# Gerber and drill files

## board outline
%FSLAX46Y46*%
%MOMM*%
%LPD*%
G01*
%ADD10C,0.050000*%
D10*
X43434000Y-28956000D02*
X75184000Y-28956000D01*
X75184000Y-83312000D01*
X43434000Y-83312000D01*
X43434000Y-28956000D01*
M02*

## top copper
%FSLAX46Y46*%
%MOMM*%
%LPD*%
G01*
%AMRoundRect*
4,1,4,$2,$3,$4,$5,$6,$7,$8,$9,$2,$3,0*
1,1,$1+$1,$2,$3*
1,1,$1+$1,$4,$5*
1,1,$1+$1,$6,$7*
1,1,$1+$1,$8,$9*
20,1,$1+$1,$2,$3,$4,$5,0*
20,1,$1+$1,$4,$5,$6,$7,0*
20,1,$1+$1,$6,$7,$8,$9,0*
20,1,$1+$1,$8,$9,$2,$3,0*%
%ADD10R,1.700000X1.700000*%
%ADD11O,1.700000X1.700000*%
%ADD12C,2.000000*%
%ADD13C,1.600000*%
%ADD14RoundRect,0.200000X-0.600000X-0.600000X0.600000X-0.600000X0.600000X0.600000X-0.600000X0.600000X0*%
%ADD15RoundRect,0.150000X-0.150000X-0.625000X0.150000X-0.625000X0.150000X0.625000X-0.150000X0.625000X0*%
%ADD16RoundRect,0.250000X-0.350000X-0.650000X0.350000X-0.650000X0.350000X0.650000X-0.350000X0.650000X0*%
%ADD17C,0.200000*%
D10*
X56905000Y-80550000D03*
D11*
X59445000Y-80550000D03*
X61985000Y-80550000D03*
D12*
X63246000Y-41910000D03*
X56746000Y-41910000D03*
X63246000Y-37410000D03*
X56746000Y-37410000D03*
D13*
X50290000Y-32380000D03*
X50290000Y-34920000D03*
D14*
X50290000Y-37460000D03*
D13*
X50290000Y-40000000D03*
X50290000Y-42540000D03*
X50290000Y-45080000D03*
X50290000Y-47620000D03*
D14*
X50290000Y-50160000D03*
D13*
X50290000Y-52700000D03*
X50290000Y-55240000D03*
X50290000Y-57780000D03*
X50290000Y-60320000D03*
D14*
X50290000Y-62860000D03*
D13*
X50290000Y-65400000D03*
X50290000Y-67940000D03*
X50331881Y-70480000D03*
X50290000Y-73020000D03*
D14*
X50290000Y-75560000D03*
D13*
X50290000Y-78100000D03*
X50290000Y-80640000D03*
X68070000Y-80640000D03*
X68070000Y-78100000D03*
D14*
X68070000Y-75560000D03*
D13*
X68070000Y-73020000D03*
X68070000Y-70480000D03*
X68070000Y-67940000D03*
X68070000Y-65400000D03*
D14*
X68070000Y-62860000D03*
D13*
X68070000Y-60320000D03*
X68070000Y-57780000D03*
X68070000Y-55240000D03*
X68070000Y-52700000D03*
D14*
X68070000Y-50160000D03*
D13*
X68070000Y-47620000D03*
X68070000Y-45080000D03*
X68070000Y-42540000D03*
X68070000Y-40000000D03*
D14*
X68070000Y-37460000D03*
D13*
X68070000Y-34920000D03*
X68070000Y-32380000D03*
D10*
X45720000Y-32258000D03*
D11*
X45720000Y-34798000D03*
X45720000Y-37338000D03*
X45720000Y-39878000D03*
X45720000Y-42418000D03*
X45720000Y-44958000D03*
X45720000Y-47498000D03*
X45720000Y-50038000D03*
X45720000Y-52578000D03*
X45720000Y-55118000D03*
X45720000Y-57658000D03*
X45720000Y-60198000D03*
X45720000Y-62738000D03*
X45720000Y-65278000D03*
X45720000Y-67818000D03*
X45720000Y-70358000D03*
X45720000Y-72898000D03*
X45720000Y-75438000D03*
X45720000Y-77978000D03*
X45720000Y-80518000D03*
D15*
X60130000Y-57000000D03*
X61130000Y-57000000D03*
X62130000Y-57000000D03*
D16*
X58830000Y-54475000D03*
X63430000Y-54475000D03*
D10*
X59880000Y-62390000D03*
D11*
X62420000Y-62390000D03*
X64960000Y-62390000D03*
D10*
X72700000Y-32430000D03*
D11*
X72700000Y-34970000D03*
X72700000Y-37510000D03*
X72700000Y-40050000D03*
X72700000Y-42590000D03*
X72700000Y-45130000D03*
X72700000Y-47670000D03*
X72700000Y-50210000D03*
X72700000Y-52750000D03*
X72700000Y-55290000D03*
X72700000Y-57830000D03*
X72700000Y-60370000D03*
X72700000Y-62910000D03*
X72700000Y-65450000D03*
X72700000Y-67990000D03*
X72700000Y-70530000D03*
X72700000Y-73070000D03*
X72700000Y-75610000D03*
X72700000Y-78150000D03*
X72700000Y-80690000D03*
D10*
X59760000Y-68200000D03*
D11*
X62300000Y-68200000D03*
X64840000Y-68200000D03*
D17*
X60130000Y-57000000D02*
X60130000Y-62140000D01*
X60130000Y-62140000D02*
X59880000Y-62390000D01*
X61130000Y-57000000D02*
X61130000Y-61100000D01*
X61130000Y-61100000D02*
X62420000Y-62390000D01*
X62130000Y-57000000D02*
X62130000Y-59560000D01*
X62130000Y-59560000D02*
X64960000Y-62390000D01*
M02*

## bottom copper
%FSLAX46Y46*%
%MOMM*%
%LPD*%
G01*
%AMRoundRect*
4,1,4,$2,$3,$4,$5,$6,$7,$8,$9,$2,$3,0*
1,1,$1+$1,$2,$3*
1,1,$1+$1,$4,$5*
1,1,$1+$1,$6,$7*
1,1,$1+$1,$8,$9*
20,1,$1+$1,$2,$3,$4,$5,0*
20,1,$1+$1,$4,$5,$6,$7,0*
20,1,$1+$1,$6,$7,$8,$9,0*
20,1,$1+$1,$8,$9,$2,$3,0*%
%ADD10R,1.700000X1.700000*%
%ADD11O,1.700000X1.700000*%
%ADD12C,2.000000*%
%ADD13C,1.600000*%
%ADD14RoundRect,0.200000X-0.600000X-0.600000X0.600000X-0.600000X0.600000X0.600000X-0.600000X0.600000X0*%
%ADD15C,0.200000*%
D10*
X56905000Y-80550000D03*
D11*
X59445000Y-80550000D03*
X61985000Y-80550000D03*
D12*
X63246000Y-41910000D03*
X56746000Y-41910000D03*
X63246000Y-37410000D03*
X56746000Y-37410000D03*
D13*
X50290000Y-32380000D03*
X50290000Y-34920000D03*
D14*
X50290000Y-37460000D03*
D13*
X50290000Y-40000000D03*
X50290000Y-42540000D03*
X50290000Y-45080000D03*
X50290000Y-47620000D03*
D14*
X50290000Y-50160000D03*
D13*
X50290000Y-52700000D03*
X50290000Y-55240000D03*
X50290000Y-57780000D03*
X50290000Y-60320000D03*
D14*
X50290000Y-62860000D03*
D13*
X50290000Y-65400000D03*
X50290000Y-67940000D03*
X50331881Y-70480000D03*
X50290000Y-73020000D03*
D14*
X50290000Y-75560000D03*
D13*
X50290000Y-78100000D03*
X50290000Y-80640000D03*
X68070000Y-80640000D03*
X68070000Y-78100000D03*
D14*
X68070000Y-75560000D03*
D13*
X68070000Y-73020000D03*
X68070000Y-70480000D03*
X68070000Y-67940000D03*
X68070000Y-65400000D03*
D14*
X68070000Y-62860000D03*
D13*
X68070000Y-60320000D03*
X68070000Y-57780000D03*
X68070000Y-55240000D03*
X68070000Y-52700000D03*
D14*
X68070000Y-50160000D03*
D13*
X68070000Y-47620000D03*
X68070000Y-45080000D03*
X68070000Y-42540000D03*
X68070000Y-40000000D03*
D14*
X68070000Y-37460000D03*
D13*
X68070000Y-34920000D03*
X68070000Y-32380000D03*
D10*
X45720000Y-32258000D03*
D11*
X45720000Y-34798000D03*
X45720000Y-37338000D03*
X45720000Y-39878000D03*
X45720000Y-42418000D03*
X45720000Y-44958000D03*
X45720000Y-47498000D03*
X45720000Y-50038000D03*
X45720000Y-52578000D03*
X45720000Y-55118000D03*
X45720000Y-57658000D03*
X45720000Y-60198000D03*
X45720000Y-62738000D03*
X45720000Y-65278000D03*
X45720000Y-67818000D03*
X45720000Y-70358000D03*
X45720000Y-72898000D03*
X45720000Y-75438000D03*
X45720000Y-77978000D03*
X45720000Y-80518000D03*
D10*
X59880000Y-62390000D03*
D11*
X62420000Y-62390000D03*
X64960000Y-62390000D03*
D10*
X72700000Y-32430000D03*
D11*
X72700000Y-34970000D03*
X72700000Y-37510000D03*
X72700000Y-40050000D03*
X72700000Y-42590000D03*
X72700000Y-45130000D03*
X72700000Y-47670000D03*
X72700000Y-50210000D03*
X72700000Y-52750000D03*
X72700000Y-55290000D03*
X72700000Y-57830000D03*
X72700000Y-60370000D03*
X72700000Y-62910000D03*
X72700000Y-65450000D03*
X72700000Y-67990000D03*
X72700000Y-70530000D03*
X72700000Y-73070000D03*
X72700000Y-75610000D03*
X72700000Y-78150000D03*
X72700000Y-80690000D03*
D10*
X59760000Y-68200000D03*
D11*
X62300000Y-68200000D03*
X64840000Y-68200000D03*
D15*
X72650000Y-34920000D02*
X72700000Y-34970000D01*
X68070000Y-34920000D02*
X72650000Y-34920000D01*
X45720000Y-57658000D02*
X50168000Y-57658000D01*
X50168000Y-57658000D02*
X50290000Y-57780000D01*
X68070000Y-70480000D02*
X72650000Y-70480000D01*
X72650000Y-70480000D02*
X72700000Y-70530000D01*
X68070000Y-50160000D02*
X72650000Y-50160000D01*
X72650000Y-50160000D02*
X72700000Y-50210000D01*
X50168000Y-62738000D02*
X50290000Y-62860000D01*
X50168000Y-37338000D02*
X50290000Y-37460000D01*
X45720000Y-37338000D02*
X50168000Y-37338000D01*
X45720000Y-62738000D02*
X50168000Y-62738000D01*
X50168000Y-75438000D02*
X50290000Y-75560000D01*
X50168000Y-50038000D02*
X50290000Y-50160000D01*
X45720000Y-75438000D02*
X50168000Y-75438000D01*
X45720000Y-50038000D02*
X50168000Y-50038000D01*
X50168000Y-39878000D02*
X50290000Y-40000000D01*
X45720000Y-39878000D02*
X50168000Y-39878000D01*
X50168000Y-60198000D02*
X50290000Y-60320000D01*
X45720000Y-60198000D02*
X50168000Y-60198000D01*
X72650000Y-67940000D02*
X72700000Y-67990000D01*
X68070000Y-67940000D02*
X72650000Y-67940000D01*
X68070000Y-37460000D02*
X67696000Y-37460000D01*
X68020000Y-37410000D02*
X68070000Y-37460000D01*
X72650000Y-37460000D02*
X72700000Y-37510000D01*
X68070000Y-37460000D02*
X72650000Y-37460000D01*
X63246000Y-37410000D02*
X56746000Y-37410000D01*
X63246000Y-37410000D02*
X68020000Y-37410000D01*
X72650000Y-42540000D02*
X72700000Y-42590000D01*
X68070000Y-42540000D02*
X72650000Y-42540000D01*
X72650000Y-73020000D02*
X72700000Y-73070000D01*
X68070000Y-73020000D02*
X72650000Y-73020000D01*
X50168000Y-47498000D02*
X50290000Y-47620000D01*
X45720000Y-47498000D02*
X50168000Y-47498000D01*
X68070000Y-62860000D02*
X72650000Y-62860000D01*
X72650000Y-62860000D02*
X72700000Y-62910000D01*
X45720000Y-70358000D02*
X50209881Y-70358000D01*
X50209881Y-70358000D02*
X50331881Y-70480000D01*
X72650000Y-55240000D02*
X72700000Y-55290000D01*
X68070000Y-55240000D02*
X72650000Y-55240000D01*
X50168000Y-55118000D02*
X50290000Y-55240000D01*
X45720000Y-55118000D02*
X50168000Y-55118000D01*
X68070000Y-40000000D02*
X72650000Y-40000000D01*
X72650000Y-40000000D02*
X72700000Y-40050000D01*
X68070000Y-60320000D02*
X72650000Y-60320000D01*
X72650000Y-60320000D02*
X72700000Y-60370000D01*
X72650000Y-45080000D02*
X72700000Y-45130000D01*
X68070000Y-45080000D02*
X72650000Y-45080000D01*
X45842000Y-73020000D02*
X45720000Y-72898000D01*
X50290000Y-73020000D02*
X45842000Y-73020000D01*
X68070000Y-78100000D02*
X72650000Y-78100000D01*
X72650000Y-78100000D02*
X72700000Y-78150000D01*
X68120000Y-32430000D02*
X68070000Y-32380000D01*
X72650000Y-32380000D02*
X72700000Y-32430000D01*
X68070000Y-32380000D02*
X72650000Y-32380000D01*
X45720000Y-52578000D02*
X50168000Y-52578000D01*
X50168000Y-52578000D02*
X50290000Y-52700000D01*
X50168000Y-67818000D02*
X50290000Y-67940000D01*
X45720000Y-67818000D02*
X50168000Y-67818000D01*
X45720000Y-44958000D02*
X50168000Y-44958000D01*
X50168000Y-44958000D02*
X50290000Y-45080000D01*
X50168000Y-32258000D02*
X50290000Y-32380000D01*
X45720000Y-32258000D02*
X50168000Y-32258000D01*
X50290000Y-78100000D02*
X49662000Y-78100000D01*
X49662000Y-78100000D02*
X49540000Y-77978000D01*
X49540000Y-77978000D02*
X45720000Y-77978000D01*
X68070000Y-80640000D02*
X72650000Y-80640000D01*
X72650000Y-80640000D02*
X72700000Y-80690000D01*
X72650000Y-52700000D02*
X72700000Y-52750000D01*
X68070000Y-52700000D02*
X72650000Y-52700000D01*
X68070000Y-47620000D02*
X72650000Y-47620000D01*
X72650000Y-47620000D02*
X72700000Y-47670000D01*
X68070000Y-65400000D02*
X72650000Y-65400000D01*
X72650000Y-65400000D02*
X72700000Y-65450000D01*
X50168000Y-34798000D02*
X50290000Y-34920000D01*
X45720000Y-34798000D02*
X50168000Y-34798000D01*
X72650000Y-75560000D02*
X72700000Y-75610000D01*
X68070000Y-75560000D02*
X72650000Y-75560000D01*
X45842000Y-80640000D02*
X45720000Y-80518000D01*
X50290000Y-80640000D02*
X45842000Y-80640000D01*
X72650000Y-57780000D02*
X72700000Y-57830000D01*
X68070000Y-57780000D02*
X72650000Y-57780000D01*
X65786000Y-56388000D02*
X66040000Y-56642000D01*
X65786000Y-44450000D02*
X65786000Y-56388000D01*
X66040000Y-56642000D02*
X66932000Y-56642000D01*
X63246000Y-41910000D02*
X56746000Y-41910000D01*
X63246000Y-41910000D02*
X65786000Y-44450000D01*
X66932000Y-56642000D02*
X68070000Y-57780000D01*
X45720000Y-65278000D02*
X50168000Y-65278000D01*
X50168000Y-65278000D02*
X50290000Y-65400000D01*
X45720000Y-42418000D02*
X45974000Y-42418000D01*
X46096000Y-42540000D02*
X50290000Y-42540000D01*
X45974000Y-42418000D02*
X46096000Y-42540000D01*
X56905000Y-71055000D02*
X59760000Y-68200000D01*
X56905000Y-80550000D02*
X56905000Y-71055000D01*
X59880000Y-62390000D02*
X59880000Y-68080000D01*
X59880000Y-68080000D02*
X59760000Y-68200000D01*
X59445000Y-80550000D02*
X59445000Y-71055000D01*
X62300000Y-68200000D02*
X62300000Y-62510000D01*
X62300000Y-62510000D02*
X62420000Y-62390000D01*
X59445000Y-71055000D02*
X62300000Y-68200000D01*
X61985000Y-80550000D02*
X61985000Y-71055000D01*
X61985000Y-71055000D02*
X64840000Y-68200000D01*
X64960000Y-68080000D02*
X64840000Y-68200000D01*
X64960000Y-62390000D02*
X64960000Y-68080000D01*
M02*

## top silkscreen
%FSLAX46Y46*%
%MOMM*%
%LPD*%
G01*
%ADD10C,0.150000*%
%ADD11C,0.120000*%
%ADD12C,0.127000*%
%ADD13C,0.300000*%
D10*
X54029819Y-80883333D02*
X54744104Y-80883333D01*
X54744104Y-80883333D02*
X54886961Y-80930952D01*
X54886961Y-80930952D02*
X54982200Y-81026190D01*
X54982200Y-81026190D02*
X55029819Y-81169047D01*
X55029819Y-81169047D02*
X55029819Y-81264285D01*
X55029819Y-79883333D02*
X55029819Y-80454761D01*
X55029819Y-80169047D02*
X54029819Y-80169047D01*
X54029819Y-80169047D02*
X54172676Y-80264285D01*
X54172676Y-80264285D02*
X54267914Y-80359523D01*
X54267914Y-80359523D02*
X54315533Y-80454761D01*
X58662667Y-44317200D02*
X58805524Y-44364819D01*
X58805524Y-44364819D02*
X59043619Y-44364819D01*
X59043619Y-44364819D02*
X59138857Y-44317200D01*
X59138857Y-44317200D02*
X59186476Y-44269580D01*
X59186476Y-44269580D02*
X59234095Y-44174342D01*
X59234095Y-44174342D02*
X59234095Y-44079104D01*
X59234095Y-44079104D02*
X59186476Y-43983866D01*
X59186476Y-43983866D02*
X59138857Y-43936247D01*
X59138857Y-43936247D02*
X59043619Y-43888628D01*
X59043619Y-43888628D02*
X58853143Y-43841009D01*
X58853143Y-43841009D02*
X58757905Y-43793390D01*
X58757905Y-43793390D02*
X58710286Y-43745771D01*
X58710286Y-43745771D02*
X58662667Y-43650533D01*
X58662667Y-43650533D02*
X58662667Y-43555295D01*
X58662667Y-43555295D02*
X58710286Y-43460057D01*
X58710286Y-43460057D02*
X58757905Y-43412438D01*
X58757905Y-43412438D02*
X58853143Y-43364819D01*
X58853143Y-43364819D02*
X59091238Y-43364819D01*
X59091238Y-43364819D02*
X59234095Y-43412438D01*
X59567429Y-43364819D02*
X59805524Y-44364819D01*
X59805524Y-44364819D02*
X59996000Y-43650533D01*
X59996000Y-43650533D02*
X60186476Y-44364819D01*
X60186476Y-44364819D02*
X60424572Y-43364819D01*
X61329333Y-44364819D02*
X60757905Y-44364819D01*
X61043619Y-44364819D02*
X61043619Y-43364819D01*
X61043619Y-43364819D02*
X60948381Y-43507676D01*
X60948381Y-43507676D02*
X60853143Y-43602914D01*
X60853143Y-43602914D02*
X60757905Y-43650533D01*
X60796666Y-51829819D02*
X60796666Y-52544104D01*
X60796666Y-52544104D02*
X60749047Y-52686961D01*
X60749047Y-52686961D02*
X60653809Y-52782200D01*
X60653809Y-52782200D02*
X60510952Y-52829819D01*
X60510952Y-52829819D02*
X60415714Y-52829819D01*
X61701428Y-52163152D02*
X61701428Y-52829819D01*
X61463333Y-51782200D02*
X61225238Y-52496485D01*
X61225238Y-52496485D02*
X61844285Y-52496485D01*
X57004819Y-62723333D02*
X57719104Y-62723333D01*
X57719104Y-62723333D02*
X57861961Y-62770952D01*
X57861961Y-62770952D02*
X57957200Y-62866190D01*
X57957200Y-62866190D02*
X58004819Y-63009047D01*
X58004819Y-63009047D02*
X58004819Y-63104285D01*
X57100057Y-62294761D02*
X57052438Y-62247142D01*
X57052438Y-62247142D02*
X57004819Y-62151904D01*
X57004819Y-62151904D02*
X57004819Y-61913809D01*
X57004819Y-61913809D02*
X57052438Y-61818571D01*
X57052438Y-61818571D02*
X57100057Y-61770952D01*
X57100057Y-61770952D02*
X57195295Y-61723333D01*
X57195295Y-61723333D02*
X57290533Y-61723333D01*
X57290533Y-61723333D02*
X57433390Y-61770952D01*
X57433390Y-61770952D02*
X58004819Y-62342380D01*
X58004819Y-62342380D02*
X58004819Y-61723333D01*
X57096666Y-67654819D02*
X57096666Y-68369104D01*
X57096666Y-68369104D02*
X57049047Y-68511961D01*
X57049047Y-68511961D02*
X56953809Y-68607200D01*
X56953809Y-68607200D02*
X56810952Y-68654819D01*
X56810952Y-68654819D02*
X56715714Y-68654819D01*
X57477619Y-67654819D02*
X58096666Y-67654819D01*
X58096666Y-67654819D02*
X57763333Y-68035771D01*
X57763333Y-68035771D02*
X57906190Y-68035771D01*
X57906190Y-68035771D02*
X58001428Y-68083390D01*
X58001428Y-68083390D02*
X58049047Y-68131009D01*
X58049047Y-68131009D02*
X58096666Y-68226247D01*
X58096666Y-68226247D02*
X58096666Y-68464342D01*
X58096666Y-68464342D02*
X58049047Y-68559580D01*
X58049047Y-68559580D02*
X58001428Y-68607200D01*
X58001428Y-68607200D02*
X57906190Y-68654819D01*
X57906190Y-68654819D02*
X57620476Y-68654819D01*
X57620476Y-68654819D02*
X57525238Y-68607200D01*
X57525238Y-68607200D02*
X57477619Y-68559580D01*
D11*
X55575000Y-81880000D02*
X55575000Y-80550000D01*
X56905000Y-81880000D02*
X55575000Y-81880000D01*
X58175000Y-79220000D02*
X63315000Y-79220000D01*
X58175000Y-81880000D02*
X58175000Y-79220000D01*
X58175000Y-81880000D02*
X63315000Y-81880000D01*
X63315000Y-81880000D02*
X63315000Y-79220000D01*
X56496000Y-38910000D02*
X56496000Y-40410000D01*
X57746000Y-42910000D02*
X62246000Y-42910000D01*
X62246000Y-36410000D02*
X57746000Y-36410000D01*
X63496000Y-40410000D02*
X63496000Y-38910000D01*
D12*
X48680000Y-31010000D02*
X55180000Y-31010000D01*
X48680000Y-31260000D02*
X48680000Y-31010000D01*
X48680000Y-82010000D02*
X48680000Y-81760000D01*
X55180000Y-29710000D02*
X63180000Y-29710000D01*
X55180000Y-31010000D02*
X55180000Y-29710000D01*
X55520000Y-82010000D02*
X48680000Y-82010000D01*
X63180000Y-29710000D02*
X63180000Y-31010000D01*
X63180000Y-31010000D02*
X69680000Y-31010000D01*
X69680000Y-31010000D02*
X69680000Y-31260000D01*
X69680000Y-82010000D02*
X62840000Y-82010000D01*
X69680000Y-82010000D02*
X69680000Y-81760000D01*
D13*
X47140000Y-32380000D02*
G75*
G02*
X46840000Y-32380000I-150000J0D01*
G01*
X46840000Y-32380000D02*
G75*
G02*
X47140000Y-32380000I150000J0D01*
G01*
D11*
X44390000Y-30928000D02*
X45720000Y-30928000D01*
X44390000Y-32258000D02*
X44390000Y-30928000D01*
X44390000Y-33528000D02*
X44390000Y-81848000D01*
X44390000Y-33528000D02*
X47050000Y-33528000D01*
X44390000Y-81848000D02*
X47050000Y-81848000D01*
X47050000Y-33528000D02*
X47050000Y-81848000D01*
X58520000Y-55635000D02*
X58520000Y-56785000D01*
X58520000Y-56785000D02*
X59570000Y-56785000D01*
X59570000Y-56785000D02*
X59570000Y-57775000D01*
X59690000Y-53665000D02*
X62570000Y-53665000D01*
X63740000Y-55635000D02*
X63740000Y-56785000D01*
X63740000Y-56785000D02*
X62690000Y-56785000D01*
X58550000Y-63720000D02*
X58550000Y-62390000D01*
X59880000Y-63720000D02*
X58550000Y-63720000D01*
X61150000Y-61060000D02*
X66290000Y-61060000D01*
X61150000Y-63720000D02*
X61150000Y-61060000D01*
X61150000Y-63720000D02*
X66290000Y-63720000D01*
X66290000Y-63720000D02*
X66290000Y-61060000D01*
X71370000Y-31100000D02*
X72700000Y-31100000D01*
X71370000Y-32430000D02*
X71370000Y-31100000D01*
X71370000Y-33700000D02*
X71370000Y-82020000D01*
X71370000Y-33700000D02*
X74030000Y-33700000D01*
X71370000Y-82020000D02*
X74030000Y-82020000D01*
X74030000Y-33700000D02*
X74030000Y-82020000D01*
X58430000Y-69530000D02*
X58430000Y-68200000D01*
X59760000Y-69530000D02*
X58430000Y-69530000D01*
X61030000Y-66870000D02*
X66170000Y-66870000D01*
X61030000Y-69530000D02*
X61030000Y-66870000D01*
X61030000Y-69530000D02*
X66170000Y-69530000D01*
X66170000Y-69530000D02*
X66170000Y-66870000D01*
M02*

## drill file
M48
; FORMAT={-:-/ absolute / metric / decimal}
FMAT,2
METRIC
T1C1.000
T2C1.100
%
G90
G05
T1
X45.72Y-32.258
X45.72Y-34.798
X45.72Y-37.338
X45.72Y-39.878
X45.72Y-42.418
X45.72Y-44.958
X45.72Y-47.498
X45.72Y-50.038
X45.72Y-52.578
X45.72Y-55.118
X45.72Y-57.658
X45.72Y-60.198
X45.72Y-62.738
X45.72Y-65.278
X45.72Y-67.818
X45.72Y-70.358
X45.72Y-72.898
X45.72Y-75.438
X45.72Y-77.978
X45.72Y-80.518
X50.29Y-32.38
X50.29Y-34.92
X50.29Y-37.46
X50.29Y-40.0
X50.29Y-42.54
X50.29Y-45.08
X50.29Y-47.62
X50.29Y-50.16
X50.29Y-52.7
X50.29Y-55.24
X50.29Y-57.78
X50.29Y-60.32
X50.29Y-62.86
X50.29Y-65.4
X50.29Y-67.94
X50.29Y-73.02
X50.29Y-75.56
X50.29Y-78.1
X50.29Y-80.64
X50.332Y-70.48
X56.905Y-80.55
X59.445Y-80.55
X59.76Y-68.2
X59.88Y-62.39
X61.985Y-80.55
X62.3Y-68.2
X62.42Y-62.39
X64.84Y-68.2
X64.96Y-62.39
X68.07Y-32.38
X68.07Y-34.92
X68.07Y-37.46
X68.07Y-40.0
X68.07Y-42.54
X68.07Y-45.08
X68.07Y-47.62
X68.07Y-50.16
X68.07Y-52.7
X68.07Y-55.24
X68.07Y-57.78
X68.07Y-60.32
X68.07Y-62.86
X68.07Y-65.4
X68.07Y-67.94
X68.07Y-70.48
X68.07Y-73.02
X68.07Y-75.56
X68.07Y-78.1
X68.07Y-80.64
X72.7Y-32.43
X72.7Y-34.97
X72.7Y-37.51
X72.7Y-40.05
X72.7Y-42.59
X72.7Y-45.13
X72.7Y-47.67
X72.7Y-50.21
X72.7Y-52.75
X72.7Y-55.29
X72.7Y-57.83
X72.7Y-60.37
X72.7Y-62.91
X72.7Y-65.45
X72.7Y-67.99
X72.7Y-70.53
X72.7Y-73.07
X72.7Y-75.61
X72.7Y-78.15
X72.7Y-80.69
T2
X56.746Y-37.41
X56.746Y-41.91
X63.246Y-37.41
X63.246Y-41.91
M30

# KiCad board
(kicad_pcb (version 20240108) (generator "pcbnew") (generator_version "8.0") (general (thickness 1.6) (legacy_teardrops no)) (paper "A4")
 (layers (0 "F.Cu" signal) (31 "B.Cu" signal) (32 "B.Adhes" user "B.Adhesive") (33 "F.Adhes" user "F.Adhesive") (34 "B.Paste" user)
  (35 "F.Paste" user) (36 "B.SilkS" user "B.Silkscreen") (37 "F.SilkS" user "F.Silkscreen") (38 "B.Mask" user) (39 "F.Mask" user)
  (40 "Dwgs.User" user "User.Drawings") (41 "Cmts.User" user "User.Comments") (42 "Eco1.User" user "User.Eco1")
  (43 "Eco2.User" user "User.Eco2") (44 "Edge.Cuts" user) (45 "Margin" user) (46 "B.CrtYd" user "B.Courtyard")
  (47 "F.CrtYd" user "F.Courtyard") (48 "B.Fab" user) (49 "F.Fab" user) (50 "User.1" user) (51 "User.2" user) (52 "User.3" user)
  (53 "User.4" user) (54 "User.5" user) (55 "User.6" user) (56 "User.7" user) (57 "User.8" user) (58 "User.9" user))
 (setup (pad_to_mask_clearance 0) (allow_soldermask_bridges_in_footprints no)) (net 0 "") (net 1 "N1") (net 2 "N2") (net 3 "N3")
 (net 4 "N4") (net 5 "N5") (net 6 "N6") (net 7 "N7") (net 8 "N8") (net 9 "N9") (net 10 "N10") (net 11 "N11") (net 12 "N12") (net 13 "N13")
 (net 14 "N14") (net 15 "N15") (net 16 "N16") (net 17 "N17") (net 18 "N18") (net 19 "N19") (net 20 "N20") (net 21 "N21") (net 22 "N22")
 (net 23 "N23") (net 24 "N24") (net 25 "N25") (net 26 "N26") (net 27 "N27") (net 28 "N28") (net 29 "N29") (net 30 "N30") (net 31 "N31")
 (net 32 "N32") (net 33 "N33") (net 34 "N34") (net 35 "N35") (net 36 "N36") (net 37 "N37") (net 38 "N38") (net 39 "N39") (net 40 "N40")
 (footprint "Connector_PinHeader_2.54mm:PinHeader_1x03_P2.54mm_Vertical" (layer "F.Cu") (at 56.905 80.55 90)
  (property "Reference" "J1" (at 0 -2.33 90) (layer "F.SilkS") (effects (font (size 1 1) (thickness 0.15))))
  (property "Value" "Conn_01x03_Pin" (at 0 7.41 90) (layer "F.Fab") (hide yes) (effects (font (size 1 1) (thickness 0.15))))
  (fp_line (start -1.33 -1.33) (end 0 -1.33) (stroke (width 0.12) (type solid)) (layer "F.SilkS"))
  (fp_line (start -1.33 0) (end -1.33 -1.33) (stroke (width 0.12) (type solid)) (layer "F.SilkS"))
  (fp_line (start 1.33 1.27) (end 1.33 6.41) (stroke (width 0.12) (type solid)) (layer "F.SilkS"))
  (fp_line (start -1.33 1.27) (end 1.33 1.27) (stroke (width 0.12) (type solid)) (layer "F.SilkS"))
  (fp_line (start -1.33 1.27) (end -1.33 6.41) (stroke (width 0.12) (type solid)) (layer "F.SilkS"))
  (fp_line (start -1.33 6.41) (end 1.33 6.41) (stroke (width 0.12) (type solid)) (layer "F.SilkS"))
  (pad "1" thru_hole rect (at 0 0 90) (size 1.7 1.7) (drill 1) (layers "*.Cu" "*.Mask") (remove_unused_layers no) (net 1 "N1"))
  (pad "2" thru_hole oval (at 0 2.54 90) (size 1.7 1.7) (drill 1) (layers "*.Cu" "*.Mask") (remove_unused_layers no) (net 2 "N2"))
  (pad "3" thru_hole oval (at 0 5.08 90) (size 1.7 1.7) (drill 1) (layers "*.Cu" "*.Mask") (remove_unused_layers no) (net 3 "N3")))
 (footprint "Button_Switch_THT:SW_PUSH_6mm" (layer "F.Cu") (at 63.246 41.91 180)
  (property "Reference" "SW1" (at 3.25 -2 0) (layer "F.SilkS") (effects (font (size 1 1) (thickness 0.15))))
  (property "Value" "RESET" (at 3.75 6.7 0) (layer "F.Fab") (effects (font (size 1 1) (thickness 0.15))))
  (fp_line (start 6.75 3) (end 6.75 1.5) (stroke (width 0.12) (type solid)) (layer "F.SilkS"))
  (fp_line (start 5.5 -1) (end 1 -1) (stroke (width 0.12) (type solid)) (layer "F.SilkS"))
  (fp_line (start 1 5.5) (end 5.5 5.5) (stroke (width 0.12) (type solid)) (layer "F.SilkS"))
  (fp_line (start -0.25 1.5) (end -0.25 3) (stroke (width 0.12) (type solid)) (layer "F.SilkS"))
  (pad "1" thru_hole circle (at 0 0 270) (size 2 2) (drill 1.1) (layers "*.Cu" "*.Mask") (remove_unused_layers no) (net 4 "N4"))
  (pad "1" thru_hole circle (at 6.5 0 270) (size 2 2) (drill 1.1) (layers "*.Cu" "*.Mask") (remove_unused_layers no) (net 4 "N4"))
  (pad "2" thru_hole circle (at 0 4.5 270) (size 2 2) (drill 1.1) (layers "*.Cu" "*.Mask") (remove_unused_layers no) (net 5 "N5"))
  (pad "2" thru_hole circle (at 6.5 4.5 270) (size 2 2) (drill 1.1) (layers "*.Cu" "*.Mask") (remove_unused_layers no) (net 5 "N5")))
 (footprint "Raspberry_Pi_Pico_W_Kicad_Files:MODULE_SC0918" (layer "F.Cu") (at 59.18 56.51)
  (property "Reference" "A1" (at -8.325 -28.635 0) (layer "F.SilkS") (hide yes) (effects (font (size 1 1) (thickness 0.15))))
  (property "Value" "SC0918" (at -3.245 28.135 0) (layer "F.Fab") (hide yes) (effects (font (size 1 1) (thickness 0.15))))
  (fp_line (start -10.5 -25.5) (end -4 -25.5) (stroke (width 0.127) (type solid)) (layer "F.SilkS"))
  (fp_line (start -10.5 -25.25) (end -10.5 -25.5) (stroke (width 0.127) (type solid)) (layer "F.SilkS"))
  (fp_line (start -10.5 25.5) (end -10.5 25.25) (stroke (width 0.127) (type solid)) (layer "F.SilkS"))
  (fp_line (start -4 -26.8) (end 4 -26.8) (stroke (width 0.127) (type solid)) (layer "F.SilkS"))
  (fp_line (start -4 -25.5) (end -4 -26.8) (stroke (width 0.127) (type solid)) (layer "F.SilkS"))
  (fp_line (start -3.66 25.5) (end -10.5 25.5) (stroke (width 0.127) (type solid)) (layer "F.SilkS"))
  (fp_line (start 4 -26.8) (end 4 -25.5) (stroke (width 0.127) (type solid)) (layer "F.SilkS"))
  (fp_line (start 4 -25.5) (end 10.5 -25.5) (stroke (width 0.127) (type solid)) (layer "F.SilkS"))
  (fp_line (start 10.5 -25.5) (end 10.5 -25.25) (stroke (width 0.127) (type solid)) (layer "F.SilkS"))
  (fp_line (start 10.5 25.5) (end 3.66 25.5) (stroke (width 0.127) (type solid)) (layer "F.SilkS"))
  (fp_line (start 10.5 25.5) (end 10.5 25.25) (stroke (width 0.127) (type solid)) (layer "F.SilkS"))
  (fp_circle (center -12.19 -24.13) (end -11.99 -24.13) (stroke (width 0.2) (type solid)) (fill solid) (layer "F.SilkS"))
  (pad "1" thru_hole circle (at -8.89 -24.13) (size 1.6 1.6) (drill 1) (layers "*.Cu" "*.Mask") (remove_unused_layers no) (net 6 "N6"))
  (pad "2" thru_hole circle (at -8.89 -21.59) (size 1.6 1.6) (drill 1) (layers "*.Cu" "*.Mask") (remove_unused_layers no) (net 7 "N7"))
  (pad "3" thru_hole roundrect (at -8.89 -19.05) (size 1.6 1.6) (drill 1) (layers "*.Cu" "*.Mask") (remove_unused_layers no)
   (roundrect_rratio 0.125) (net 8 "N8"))
  (pad "4" thru_hole circle (at -8.89 -16.51) (size 1.6 1.6) (drill 1) (layers "*.Cu" "*.Mask") (remove_unused_layers no) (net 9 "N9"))
  (pad "5" thru_hole circle (at -8.89 -13.97) (size 1.6 1.6) (drill 1) (layers "*.Cu" "*.Mask") (remove_unused_layers no) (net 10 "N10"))
  (pad "6" thru_hole circle (at -8.89 -11.43) (size 1.6 1.6) (drill 1) (layers "*.Cu" "*.Mask") (remove_unused_layers no) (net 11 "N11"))
  (pad "7" thru_hole circle (at -8.89 -8.89) (size 1.6 1.6) (drill 1) (layers "*.Cu" "*.Mask") (remove_unused_layers no) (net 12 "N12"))
  (pad "8" thru_hole roundrect (at -8.89 -6.35) (size 1.6 1.6) (drill 1) (layers "*.Cu" "*.Mask") (remove_unused_layers no)
   (roundrect_rratio 0.125) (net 8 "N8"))
  (pad "9" thru_hole circle (at -8.89 -3.81) (size 1.6 1.6) (drill 1) (layers "*.Cu" "*.Mask") (remove_unused_layers no) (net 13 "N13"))
  (pad "10" thru_hole circle (at -8.89 -1.27) (size 1.6 1.6) (drill 1) (layers "*.Cu" "*.Mask") (remove_unused_layers no) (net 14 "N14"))
  (pad "11" thru_hole circle (at -8.89 1.27) (size 1.6 1.6) (drill 1) (layers "*.Cu" "*.Mask") (remove_unused_layers no) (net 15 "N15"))
  (pad "12" thru_hole circle (at -8.89 3.81) (size 1.6 1.6) (drill 1) (layers "*.Cu" "*.Mask") (remove_unused_layers no) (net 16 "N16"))
  (pad "13" thru_hole roundrect (at -8.89 6.35) (size 1.6 1.6) (drill 1) (layers "*.Cu" "*.Mask") (remove_unused_layers no)
   (roundrect_rratio 0.125) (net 8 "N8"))
  (pad "14" thru_hole circle (at -8.89 8.89) (size 1.6 1.6) (drill 1) (layers "*.Cu" "*.Mask") (remove_unused_layers no) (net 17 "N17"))
  (pad "15" thru_hole circle (at -8.89 11.43) (size 1.6 1.6) (drill 1) (layers "*.Cu" "*.Mask") (remove_unused_layers no) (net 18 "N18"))
  (pad "16" thru_hole circle (at -8.848119 13.97) (size 1.6 1.6) (drill 1) (layers "*.Cu" "*.Mask") (remove_unused_layers no) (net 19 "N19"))
  (pad "17" thru_hole circle (at -8.89 16.51) (size 1.6 1.6) (drill 1) (layers "*.Cu" "*.Mask") (remove_unused_layers no) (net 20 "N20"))
  (pad "18" thru_hole roundrect (at -8.89 19.05) (size 1.6 1.6) (drill 1) (layers "*.Cu" "*.Mask") (remove_unused_layers no)
   (roundrect_rratio 0.125) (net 8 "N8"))
  (pad "19" thru_hole circle (at -8.89 21.59) (size 1.6 1.6) (drill 1) (layers "*.Cu" "*.Mask") (remove_unused_layers no) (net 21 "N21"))
  (pad "20" thru_hole circle (at -8.89 24.13) (size 1.6 1.6) (drill 1) (layers "*.Cu" "*.Mask") (remove_unused_layers no) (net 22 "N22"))
  (pad "21" thru_hole circle (at 8.89 24.13) (size 1.6 1.6) (drill 1) (layers "*.Cu" "*.Mask") (remove_unused_layers no) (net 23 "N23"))
  (pad "22" thru_hole circle (at 8.89 21.59) (size 1.6 1.6) (drill 1) (layers "*.Cu" "*.Mask") (remove_unused_layers no) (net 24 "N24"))
  (pad "23" thru_hole roundrect (at 8.89 19.05) (size 1.6 1.6) (drill 1) (layers "*.Cu" "*.Mask") (remove_unused_layers no)
   (roundrect_rratio 0.125) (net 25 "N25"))
  (pad "24" thru_hole circle (at 8.89 16.51) (size 1.6 1.6) (drill 1) (layers "*.Cu" "*.Mask") (remove_unused_layers no) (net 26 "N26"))
  (pad "25" thru_hole circle (at 8.89 13.97) (size 1.6 1.6) (drill 1) (layers "*.Cu" "*.Mask") (remove_unused_layers no) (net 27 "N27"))
  (pad "26" thru_hole circle (at 8.89 11.43) (size 1.6 1.6) (drill 1) (layers "*.Cu" "*.Mask") (remove_unused_layers no) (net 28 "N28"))
  (pad "27" thru_hole circle (at 8.89 8.89) (size 1.6 1.6) (drill 1) (layers "*.Cu" "*.Mask") (remove_unused_layers no) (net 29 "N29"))
  (pad "28" thru_hole roundrect (at 8.89 6.35) (size 1.6 1.6) (drill 1) (layers "*.Cu" "*.Mask") (remove_unused_layers no)
   (roundrect_rratio 0.125) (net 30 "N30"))
  (pad "29" thru_hole circle (at 8.89 3.81) (size 1.6 1.6) (drill 1) (layers "*.Cu" "*.Mask") (remove_unused_layers no) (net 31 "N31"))
  (pad "30" thru_hole circle (at 8.89 1.27) (size 1.6 1.6) (drill 1) (layers "*.Cu" "*.Mask") (remove_unused_layers no) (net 4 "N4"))
  (pad "31" thru_hole circle (at 8.89 -1.27) (size 1.6 1.6) (drill 1) (layers "*.Cu" "*.Mask") (remove_unused_layers no) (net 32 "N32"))
  (pad "32" thru_hole circle (at 8.89 -3.81) (size 1.6 1.6) (drill 1) (layers "*.Cu" "*.Mask") (remove_unused_layers no) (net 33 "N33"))
  (pad "33" thru_hole roundrect (at 8.89 -6.35) (size 1.6 1.6) (drill 1) (layers "*.Cu" "*.Mask") (remove_unused_layers no)
   (roundrect_rratio 0.125) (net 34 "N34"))
  (pad "34" thru_hole circle (at 8.89 -8.89) (size 1.6 1.6) (drill 1) (layers "*.Cu" "*.Mask") (remove_unused_layers no) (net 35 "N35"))
  (pad "35" thru_hole circle (at 8.89 -11.43) (size 1.6 1.6) (drill 1) (layers "*.Cu" "*.Mask") (remove_unused_layers no) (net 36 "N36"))
  (pad "36" thru_hole circle (at 8.89 -13.97) (size 1.6 1.6) (drill 1) (layers "*.Cu" "*.Mask") (remove_unused_layers no) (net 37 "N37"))
  (pad "37" thru_hole circle (at 8.89 -16.51) (size 1.6 1.6) (drill 1) (layers "*.Cu" "*.Mask") (remove_unused_layers no) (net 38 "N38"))
  (pad "38" thru_hole roundrect (at 8.89 -19.05) (size 1.6 1.6) (drill 1) (layers "*.Cu" "*.Mask") (remove_unused_layers no)
   (roundrect_rratio 0.125) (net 5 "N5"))
  (pad "39" thru_hole circle (at 8.89 -21.59) (size 1.6 1.6) (drill 1) (layers "*.Cu" "*.Mask") (remove_unused_layers no) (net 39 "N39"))
  (pad "40" thru_hole circle (at 8.89 -24.13) (size 1.6 1.6) (drill 1) (layers "*.Cu" "*.Mask") (remove_unused_layers no) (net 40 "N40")))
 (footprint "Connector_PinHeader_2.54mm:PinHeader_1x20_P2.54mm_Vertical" (layer "F.Cu") (at 45.72 32.258)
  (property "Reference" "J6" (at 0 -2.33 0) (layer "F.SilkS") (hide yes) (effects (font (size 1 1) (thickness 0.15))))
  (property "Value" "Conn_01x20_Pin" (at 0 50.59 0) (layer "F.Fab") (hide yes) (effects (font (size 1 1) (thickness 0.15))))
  (fp_line (start -1.33 -1.33) (end 0 -1.33) (stroke (width 0.12) (type solid)) (layer "F.SilkS"))
  (fp_line (start -1.33 0) (end -1.33 -1.33) (stroke (width 0.12) (type solid)) (layer "F.SilkS"))
  (fp_line (start -1.33 1.27) (end -1.33 49.59) (stroke (width 0.12) (type solid)) (layer "F.SilkS"))
  (fp_line (start -1.33 1.27) (end 1.33 1.27) (stroke (width 0.12) (type solid)) (layer "F.SilkS"))
  (fp_line (start -1.33 49.59) (end 1.33 49.59) (stroke (width 0.12) (type solid)) (layer "F.SilkS"))
  (fp_line (start 1.33 1.27) (end 1.33 49.59) (stroke (width 0.12) (type solid)) (layer "F.SilkS"))
  (pad "1" thru_hole rect (at 0 0) (size 1.7 1.7) (drill 1) (layers "*.Cu" "*.Mask") (remove_unused_layers no) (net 6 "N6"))
  (pad "2" thru_hole oval (at 0 2.54) (size 1.7 1.7) (drill 1) (layers "*.Cu" "*.Mask") (remove_unused_layers no) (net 7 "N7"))
  (pad "3" thru_hole oval (at 0 5.08) (size 1.7 1.7) (drill 1) (layers "*.Cu" "*.Mask") (remove_unused_layers no) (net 8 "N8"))
  (pad "4" thru_hole oval (at 0 7.62) (size 1.7 1.7) (drill 1) (layers "*.Cu" "*.Mask") (remove_unused_layers no) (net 9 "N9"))
  (pad "5" thru_hole oval (at 0 10.16) (size 1.7 1.7) (drill 1) (layers "*.Cu" "*.Mask") (remove_unused_layers no) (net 10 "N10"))
  (pad "6" thru_hole oval (at 0 12.7) (size 1.7 1.7) (drill 1) (layers "*.Cu" "*.Mask") (remove_unused_layers no) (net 11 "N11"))
  (pad "7" thru_hole oval (at 0 15.24) (size 1.7 1.7) (drill 1) (layers "*.Cu" "*.Mask") (remove_unused_layers no) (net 12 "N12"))
  (pad "8" thru_hole oval (at 0 17.78) (size 1.7 1.7) (drill 1) (layers "*.Cu" "*.Mask") (remove_unused_layers no) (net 8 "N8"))
  (pad "9" thru_hole oval (at 0 20.32) (size 1.7 1.7) (drill 1) (layers "*.Cu" "*.Mask") (remove_unused_layers no) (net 13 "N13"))
  (pad "10" thru_hole oval (at 0 22.86) (size 1.7 1.7) (drill 1) (layers "*.Cu" "*.Mask") (remove_unused_layers no) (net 14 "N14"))
  (pad "11" thru_hole oval (at 0 25.4) (size 1.7 1.7) (drill 1) (layers "*.Cu" "*.Mask") (remove_unused_layers no) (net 15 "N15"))
  (pad "12" thru_hole oval (at 0 27.94) (size 1.7 1.7) (drill 1) (layers "*.Cu" "*.Mask") (remove_unused_layers no) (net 16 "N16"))
  (pad "13" thru_hole oval (at 0 30.48) (size 1.7 1.7) (drill 1) (layers "*.Cu" "*.Mask") (remove_unused_layers no) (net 8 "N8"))
  (pad "14" thru_hole oval (at 0 33.02) (size 1.7 1.7) (drill 1) (layers "*.Cu" "*.Mask") (remove_unused_layers no) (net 17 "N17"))
  (pad "15" thru_hole oval (at 0 35.56) (size 1.7 1.7) (drill 1) (layers "*.Cu" "*.Mask") (remove_unused_layers no) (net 18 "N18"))
  (pad "16" thru_hole oval (at 0 38.1) (size 1.7 1.7) (drill 1) (layers "*.Cu" "*.Mask") (remove_unused_layers no) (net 19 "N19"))
  (pad "17" thru_hole oval (at 0 40.64) (size 1.7 1.7) (drill 1) (layers "*.Cu" "*.Mask") (remove_unused_layers no) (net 20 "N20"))
  (pad "18" thru_hole oval (at 0 43.18) (size 1.7 1.7) (drill 1) (layers "*.Cu" "*.Mask") (remove_unused_layers no) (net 8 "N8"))
  (pad "19" thru_hole oval (at 0 45.72) (size 1.7 1.7) (drill 1) (layers "*.Cu" "*.Mask") (remove_unused_layers no) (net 21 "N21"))
  (pad "20" thru_hole oval (at 0 48.26) (size 1.7 1.7) (drill 1) (layers "*.Cu" "*.Mask") (remove_unused_layers no) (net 22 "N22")))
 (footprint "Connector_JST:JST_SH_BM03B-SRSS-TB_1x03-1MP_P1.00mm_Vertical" (layer "F.Cu") (at 61.13 55.675)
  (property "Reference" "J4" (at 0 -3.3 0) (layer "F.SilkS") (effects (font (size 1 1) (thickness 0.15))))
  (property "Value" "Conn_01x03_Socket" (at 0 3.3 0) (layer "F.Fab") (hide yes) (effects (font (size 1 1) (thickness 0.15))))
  (fp_line (start -2.61 -0.04) (end -2.61 1.11) (stroke (width 0.12) (type solid)) (layer "F.SilkS"))
  (fp_line (start -2.61 1.11) (end -1.56 1.11) (stroke (width 0.12) (type solid)) (layer "F.SilkS"))
  (fp_line (start -1.56 1.11) (end -1.56 2.1) (stroke (width 0.12) (type solid)) (layer "F.SilkS"))
  (fp_line (start -1.44 -2.01) (end 1.44 -2.01) (stroke (width 0.12) (type solid)) (layer "F.SilkS"))
  (fp_line (start 2.61 -0.04) (end 2.61 1.11) (stroke (width 0.12) (type solid)) (layer "F.SilkS"))
  (fp_line (start 2.61 1.11) (end 1.56 1.11) (stroke (width 0.12) (type solid)) (layer "F.SilkS"))
  (pad "1" smd roundrect (at -1 1.325) (size 0.6 1.55) (layers "F.Cu" "F.Paste" "F.Mask") (roundrect_rratio 0.25) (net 1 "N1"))
  (pad "2" smd roundrect (at 0 1.325) (size 0.6 1.55) (layers "F.Cu" "F.Paste" "F.Mask") (roundrect_rratio 0.25) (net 2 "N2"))
  (pad "3" smd roundrect (at 1 1.325) (size 0.6 1.55) (layers "F.Cu" "F.Paste" "F.Mask") (roundrect_rratio 0.25) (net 3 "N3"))
  (pad "MP" smd roundrect (at -2.3 -1.2) (size 1.2 1.8) (layers "F.Cu" "F.Paste" "F.Mask") (roundrect_rratio 0.208333))
  (pad "MP" smd roundrect (at 2.3 -1.2) (size 1.2 1.8) (layers "F.Cu" "F.Paste" "F.Mask") (roundrect_rratio 0.208333)))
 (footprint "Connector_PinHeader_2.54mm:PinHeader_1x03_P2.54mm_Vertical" (layer "F.Cu") (at 59.88 62.39 90)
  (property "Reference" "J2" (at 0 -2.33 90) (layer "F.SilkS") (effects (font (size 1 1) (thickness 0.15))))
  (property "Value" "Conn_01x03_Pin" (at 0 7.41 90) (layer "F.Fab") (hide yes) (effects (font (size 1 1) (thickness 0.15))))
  (fp_line (start -1.33 -1.33) (end 0 -1.33) (stroke (width 0.12) (type solid)) (layer "F.SilkS"))
  (fp_line (start -1.33 0) (end -1.33 -1.33) (stroke (width 0.12) (type solid)) (layer "F.SilkS"))
  (fp_line (start 1.33 1.27) (end 1.33 6.41) (stroke (width 0.12) (type solid)) (layer "F.SilkS"))
  (fp_line (start -1.33 1.27) (end 1.33 1.27) (stroke (width 0.12) (type solid)) (layer "F.SilkS"))
  (fp_line (start -1.33 1.27) (end -1.33 6.41) (stroke (width 0.12) (type solid)) (layer "F.SilkS"))
  (fp_line (start -1.33 6.41) (end 1.33 6.41) (stroke (width 0.12) (type solid)) (layer "F.SilkS"))
  (pad "1" thru_hole rect (at 0 0 90) (size 1.7 1.7) (drill 1) (layers "*.Cu" "*.Mask") (remove_unused_layers no) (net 1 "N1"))
  (pad "2" thru_hole oval (at 0 2.54 90) (size 1.7 1.7) (drill 1) (layers "*.Cu" "*.Mask") (remove_unused_layers no) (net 2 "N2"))
  (pad "3" thru_hole oval (at 0 5.08 90) (size 1.7 1.7) (drill 1) (layers "*.Cu" "*.Mask") (remove_unused_layers no) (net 3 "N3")))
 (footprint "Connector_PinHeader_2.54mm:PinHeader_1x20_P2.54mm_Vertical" (layer "F.Cu") (at 72.7 32.43)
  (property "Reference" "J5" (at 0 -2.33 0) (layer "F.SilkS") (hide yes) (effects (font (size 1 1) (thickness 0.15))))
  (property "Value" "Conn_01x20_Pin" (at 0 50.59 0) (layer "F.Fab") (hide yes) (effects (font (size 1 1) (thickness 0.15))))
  (fp_line (start -1.33 -1.33) (end 0 -1.33) (stroke (width 0.12) (type solid)) (layer "F.SilkS"))
  (fp_line (start -1.33 0) (end -1.33 -1.33) (stroke (width 0.12) (type solid)) (layer "F.SilkS"))
  (fp_line (start -1.33 1.27) (end -1.33 49.59) (stroke (width 0.12) (type solid)) (layer "F.SilkS"))
  (fp_line (start -1.33 1.27) (end 1.33 1.27) (stroke (width 0.12) (type solid)) (layer "F.SilkS"))
  (fp_line (start -1.33 49.59) (end 1.33 49.59) (stroke (width 0.12) (type solid)) (layer "F.SilkS"))
  (fp_line (start 1.33 1.27) (end 1.33 49.59) (stroke (width 0.12) (type solid)) (layer "F.SilkS"))
  (pad "1" thru_hole rect (at 0 0) (size 1.7 1.7) (drill 1) (layers "*.Cu" "*.Mask") (remove_unused_layers no) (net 40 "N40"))
  (pad "2" thru_hole oval (at 0 2.54) (size 1.7 1.7) (drill 1) (layers "*.Cu" "*.Mask") (remove_unused_layers no) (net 39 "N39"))
  (pad "3" thru_hole oval (at 0 5.08) (size 1.7 1.7) (drill 1) (layers "*.Cu" "*.Mask") (remove_unused_layers no) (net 5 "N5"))
  (pad "4" thru_hole oval (at 0 7.62) (size 1.7 1.7) (drill 1) (layers "*.Cu" "*.Mask") (remove_unused_layers no) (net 38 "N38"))
  (pad "5" thru_hole oval (at 0 10.16) (size 1.7 1.7) (drill 1) (layers "*.Cu" "*.Mask") (remove_unused_layers no) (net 37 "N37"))
  (pad "6" thru_hole oval (at 0 12.7) (size 1.7 1.7) (drill 1) (layers "*.Cu" "*.Mask") (remove_unused_layers no) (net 36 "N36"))
  (pad "7" thru_hole oval (at 0 15.24) (size 1.7 1.7) (drill 1) (layers "*.Cu" "*.Mask") (remove_unused_layers no) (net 35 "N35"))
  (pad "8" thru_hole oval (at 0 17.78) (size 1.7 1.7) (drill 1) (layers "*.Cu" "*.Mask") (remove_unused_layers no) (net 34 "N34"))
  (pad "9" thru_hole oval (at 0 20.32) (size 1.7 1.7) (drill 1) (layers "*.Cu" "*.Mask") (remove_unused_layers no) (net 33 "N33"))
  (pad "10" thru_hole oval (at 0 22.86) (size 1.7 1.7) (drill 1) (layers "*.Cu" "*.Mask") (remove_unused_layers no) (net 32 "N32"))
  (pad "11" thru_hole oval (at 0 25.4) (size 1.7 1.7) (drill 1) (layers "*.Cu" "*.Mask") (remove_unused_layers no) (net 4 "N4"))
  (pad "12" thru_hole oval (at 0 27.94) (size 1.7 1.7) (drill 1) (layers "*.Cu" "*.Mask") (remove_unused_layers no) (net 31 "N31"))
  (pad "13" thru_hole oval (at 0 30.48) (size 1.7 1.7) (drill 1) (layers "*.Cu" "*.Mask") (remove_unused_layers no) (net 30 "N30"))
  (pad "14" thru_hole oval (at 0 33.02) (size 1.7 1.7) (drill 1) (layers "*.Cu" "*.Mask") (remove_unused_layers no) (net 29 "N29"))
  (pad "15" thru_hole oval (at 0 35.56) (size 1.7 1.7) (drill 1) (layers "*.Cu" "*.Mask") (remove_unused_layers no) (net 28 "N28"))
  (pad "16" thru_hole oval (at 0 38.1) (size 1.7 1.7) (drill 1) (layers "*.Cu" "*.Mask") (remove_unused_layers no) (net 27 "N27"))
  (pad "17" thru_hole oval (at 0 40.64) (size 1.7 1.7) (drill 1) (layers "*.Cu" "*.Mask") (remove_unused_layers no) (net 26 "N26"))
  (pad "18" thru_hole oval (at 0 43.18) (size 1.7 1.7) (drill 1) (layers "*.Cu" "*.Mask") (remove_unused_layers no) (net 25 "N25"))
  (pad "19" thru_hole oval (at 0 45.72) (size 1.7 1.7) (drill 1) (layers "*.Cu" "*.Mask") (remove_unused_layers no) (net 24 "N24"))
  (pad "20" thru_hole oval (at 0 48.26) (size 1.7 1.7) (drill 1) (layers "*.Cu" "*.Mask") (remove_unused_layers no) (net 23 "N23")))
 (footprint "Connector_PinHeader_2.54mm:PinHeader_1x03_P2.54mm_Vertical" (layer "F.Cu") (at 59.76 68.2 90)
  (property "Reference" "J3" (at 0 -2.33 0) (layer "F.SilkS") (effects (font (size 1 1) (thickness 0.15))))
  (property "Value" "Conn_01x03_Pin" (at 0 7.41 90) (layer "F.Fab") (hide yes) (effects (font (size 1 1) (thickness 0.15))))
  (fp_line (start -1.33 -1.33) (end 0 -1.33) (stroke (width 0.12) (type solid)) (layer "F.SilkS"))
  (fp_line (start -1.33 0) (end -1.33 -1.33) (stroke (width 0.12) (type solid)) (layer "F.SilkS"))
  (fp_line (start 1.33 1.27) (end 1.33 6.41) (stroke (width 0.12) (type solid)) (layer "F.SilkS"))
  (fp_line (start -1.33 1.27) (end 1.33 1.27) (stroke (width 0.12) (type solid)) (layer "F.SilkS"))
  (fp_line (start -1.33 1.27) (end -1.33 6.41) (stroke (width 0.12) (type solid)) (layer "F.SilkS"))
  (fp_line (start -1.33 6.41) (end 1.33 6.41) (stroke (width 0.12) (type solid)) (layer "F.SilkS"))
  (pad "1" thru_hole rect (at 0 0 90) (size 1.7 1.7) (drill 1) (layers "*.Cu" "*.Mask") (remove_unused_layers no) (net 1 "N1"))
  (pad "2" thru_hole oval (at 0 2.54 90) (size 1.7 1.7) (drill 1) (layers "*.Cu" "*.Mask") (remove_unused_layers no) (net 2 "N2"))
  (pad "3" thru_hole oval (at 0 5.08 90) (size 1.7 1.7) (drill 1) (layers "*.Cu" "*.Mask") (remove_unused_layers no) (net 3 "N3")))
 (gr_rect (start 43.434 28.956) (end 75.184 83.312) (stroke (width 0.05) (type default)) (fill none) (layer "Edge.Cuts"))
 (segment (start 72.65 34.92) (end 72.7 34.97) (width 0.2) (layer "B.Cu") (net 39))
 (segment (start 68.07 34.92) (end 72.65 34.92) (width 0.2) (layer "B.Cu") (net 39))
 (segment (start 45.72 57.658) (end 50.168 57.658) (width 0.2) (layer "B.Cu") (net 15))
 (segment (start 50.168 57.658) (end 50.29 57.78) (width 0.2) (layer "B.Cu") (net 15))
 (segment (start 68.07 70.48) (end 72.65 70.48) (width 0.2) (layer "B.Cu") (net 27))
 (segment (start 72.65 70.48) (end 72.7 70.53) (width 0.2) (layer "B.Cu") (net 27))
 (segment (start 68.07 50.16) (end 72.65 50.16) (width 0.2) (layer "B.Cu") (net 34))
 (segment (start 72.65 50.16) (end 72.7 50.21) (width 0.2) (layer "B.Cu") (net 34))
 (segment (start 50.168 62.738) (end 50.29 62.86) (width 0.2) (layer "B.Cu") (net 8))
 (segment (start 50.168 37.338) (end 50.29 37.46) (width 0.2) (layer "B.Cu") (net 8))
 (segment (start 45.72 37.338) (end 50.168 37.338) (width 0.2) (layer "B.Cu") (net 8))
 (segment (start 45.72 62.738) (end 50.168 62.738) (width 0.2) (layer "B.Cu") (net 8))
 (segment (start 50.168 75.438) (end 50.29 75.56) (width 0.2) (layer "B.Cu") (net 8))
 (segment (start 50.168 50.038) (end 50.29 50.16) (width 0.2) (layer "B.Cu") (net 8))
 (segment (start 45.72 75.438) (end 50.168 75.438) (width 0.2) (layer "B.Cu") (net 8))
 (segment (start 45.72 50.038) (end 50.168 50.038) (width 0.2) (layer "B.Cu") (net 8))
 (segment (start 50.168 39.878) (end 50.29 40) (width 0.2) (layer "B.Cu") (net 9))
 (segment (start 45.72 39.878) (end 50.168 39.878) (width 0.2) (layer "B.Cu") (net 9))
 (segment (start 50.168 60.198) (end 50.29 60.32) (width 0.2) (layer "B.Cu") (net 16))
 (segment (start 45.72 60.198) (end 50.168 60.198) (width 0.2) (layer "B.Cu") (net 16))
 (segment (start 72.65 67.94) (end 72.7 67.99) (width 0.2) (layer "B.Cu") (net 28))
 (segment (start 68.07 67.94) (end 72.65 67.94) (width 0.2) (layer "B.Cu") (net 28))
 (segment (start 68.07 37.46) (end 67.696 37.46) (width 0.2) (layer "B.Cu") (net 5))
 (segment (start 68.02 37.41) (end 68.07 37.46) (width 0.2) (layer "B.Cu") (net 5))
 (segment (start 72.65 37.46) (end 72.7 37.51) (width 0.2) (layer "B.Cu") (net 5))
 (segment (start 68.07 37.46) (end 72.65 37.46) (width 0.2) (layer "B.Cu") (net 5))
 (segment (start 63.246 37.41) (end 56.746 37.41) (width 0.2) (layer "B.Cu") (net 5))
 (segment (start 63.246 37.41) (end 68.02 37.41) (width 0.2) (layer "B.Cu") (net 5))
 (segment (start 72.65 42.54) (end 72.7 42.59) (width 0.2) (layer "B.Cu") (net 37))
 (segment (start 68.07 42.54) (end 72.65 42.54) (width 0.2) (layer "B.Cu") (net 37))
 (segment (start 72.65 73.02) (end 72.7 73.07) (width 0.2) (layer "B.Cu") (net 26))
 (segment (start 68.07 73.02) (end 72.65 73.02) (width 0.2) (layer "B.Cu") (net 26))
 (segment (start 50.168 47.498) (end 50.29 47.62) (width 0.2) (layer "B.Cu") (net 12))
 (segment (start 45.72 47.498) (end 50.168 47.498) (width 0.2) (layer "B.Cu") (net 12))
 (segment (start 68.07 62.86) (end 72.65 62.86) (width 0.2) (layer "B.Cu") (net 30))
 (segment (start 72.65 62.86) (end 72.7 62.91) (width 0.2) (layer "B.Cu") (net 30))
 (segment (start 45.72 70.358) (end 50.209881 70.358) (width 0.2) (layer "B.Cu") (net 19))
 (segment (start 50.209881 70.358) (end 50.331881 70.48) (width 0.2) (layer "B.Cu") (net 19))
 (segment (start 72.65 55.24) (end 72.7 55.29) (width 0.2) (layer "B.Cu") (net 32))
 (segment (start 68.07 55.24) (end 72.65 55.24) (width 0.2) (layer "B.Cu") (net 32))
 (segment (start 50.168 55.118) (end 50.29 55.24) (width 0.2) (layer "B.Cu") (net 14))
 (segment (start 45.72 55.118) (end 50.168 55.118) (width 0.2) (layer "B.Cu") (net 14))
 (segment (start 68.07 40) (end 72.65 40) (width 0.2) (layer "B.Cu") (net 38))
 (segment (start 72.65 40) (end 72.7 40.05) (width 0.2) (layer "B.Cu") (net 38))
 (segment (start 68.07 60.32) (end 72.65 60.32) (width 0.2) (layer "B.Cu") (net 31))
 (segment (start 72.65 60.32) (end 72.7 60.37) (width 0.2) (layer "B.Cu") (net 31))
 (segment (start 72.65 45.08) (end 72.7 45.13) (width 0.2) (layer "B.Cu") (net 36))
 (segment (start 68.07 45.08) (end 72.65 45.08) (width 0.2) (layer "B.Cu") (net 36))
 (segment (start 45.842 73.02) (end 45.72 72.898) (width 0.2) (layer "B.Cu") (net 20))
 (segment (start 50.29 73.02) (end 45.842 73.02) (width 0.2) (layer "B.Cu") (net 20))
 (segment (start 68.07 78.1) (end 72.65 78.1) (width 0.2) (layer "B.Cu") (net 24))
 (segment (start 72.65 78.1) (end 72.7 78.15) (width 0.2) (layer "B.Cu") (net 24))
 (segment (start 68.12 32.43) (end 68.07 32.38) (width 0.2) (layer "B.Cu") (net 40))
 (segment (start 72.65 32.38) (end 72.7 32.43) (width 0.2) (layer "B.Cu") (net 40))
 (segment (start 68.07 32.38) (end 72.65 32.38) (width 0.2) (layer "B.Cu") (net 40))
 (segment (start 45.72 52.578) (end 50.168 52.578) (width 0.2) (layer "B.Cu") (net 13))
 (segment (start 50.168 52.578) (end 50.29 52.7) (width 0.2) (layer "B.Cu") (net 13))
 (segment (start 50.168 67.818) (end 50.29 67.94) (width 0.2) (layer "B.Cu") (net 18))
 (segment (start 45.72 67.818) (end 50.168 67.818) (width 0.2) (layer "B.Cu") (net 18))
 (segment (start 45.72 44.958) (end 50.168 44.958) (width 0.2) (layer "B.Cu") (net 11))
 (segment (start 50.168 44.958) (end 50.29 45.08) (width 0.2) (layer "B.Cu") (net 11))
 (segment (start 50.168 32.258) (end 50.29 32.38) (width 0.2) (layer "B.Cu") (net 6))
 (segment (start 45.72 32.258) (end 50.168 32.258) (width 0.2) (layer "B.Cu") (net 6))
 (segment (start 50.29 78.1) (end 49.662 78.1) (width 0.2) (layer "B.Cu") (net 21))
 (segment (start 49.662 78.1) (end 49.54 77.978) (width 0.2) (layer "B.Cu") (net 21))
 (segment (start 49.54 77.978) (end 45.72 77.978) (width 0.2) (layer "B.Cu") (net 21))
 (segment (start 68.07 80.64) (end 72.65 80.64) (width 0.2) (layer "B.Cu") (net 23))
 (segment (start 72.65 80.64) (end 72.7 80.69) (width 0.2) (layer "B.Cu") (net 23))
 (segment (start 72.65 52.7) (end 72.7 52.75) (width 0.2) (layer "B.Cu") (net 33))
 (segment (start 68.07 52.7) (end 72.65 52.7) (width 0.2) (layer "B.Cu") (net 33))
 (segment (start 68.07 47.62) (end 72.65 47.62) (width 0.2) (layer "B.Cu") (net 35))
 (segment (start 72.65 47.62) (end 72.7 47.67) (width 0.2) (layer "B.Cu") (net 35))
 (segment (start 68.07 65.4) (end 72.65 65.4) (width 0.2) (layer "B.Cu") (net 29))
 (segment (start 72.65 65.4) (end 72.7 65.45) (width 0.2) (layer "B.Cu") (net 29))
 (segment (start 50.168 34.798) (end 50.29 34.92) (width 0.2) (layer "B.Cu") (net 7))
 (segment (start 45.72 34.798) (end 50.168 34.798) (width 0.2) (layer "B.Cu") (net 7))
 (segment (start 72.65 75.56) (end 72.7 75.61) (width 0.2) (layer "B.Cu") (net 25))
 (segment (start 68.07 75.56) (end 72.65 75.56) (width 0.2) (layer "B.Cu") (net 25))
 (segment (start 45.842 80.64) (end 45.72 80.518) (width 0.2) (layer "B.Cu") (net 22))
 (segment (start 50.29 80.64) (end 45.842 80.64) (width 0.2) (layer "B.Cu") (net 22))
 (segment (start 72.65 57.78) (end 72.7 57.83) (width 0.2) (layer "B.Cu") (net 4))
 (segment (start 68.07 57.78) (end 72.65 57.78) (width 0.2) (layer "B.Cu") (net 4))
 (segment (start 65.786 56.388) (end 66.04 56.642) (width 0.2) (layer "B.Cu") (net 4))
 (segment (start 65.786 44.45) (end 65.786 56.388) (width 0.2) (layer "B.Cu") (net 4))
 (segment (start 66.04 56.642) (end 66.932 56.642) (width 0.2) (layer "B.Cu") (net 4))
 (segment (start 63.246 41.91) (end 56.746 41.91) (width 0.2) (layer "B.Cu") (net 4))
 (segment (start 63.246 41.91) (end 65.786 44.45) (width 0.2) (layer "B.Cu") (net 4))
 (segment (start 66.932 56.642) (end 68.07 57.78) (width 0.2) (layer "B.Cu") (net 4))
 (segment (start 45.72 65.278) (end 50.168 65.278) (width 0.2) (layer "B.Cu") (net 17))
 (segment (start 50.168 65.278) (end 50.29 65.4) (width 0.2) (layer "B.Cu") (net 17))
 (segment (start 45.72 42.418) (end 45.974 42.418) (width 0.2) (layer "B.Cu") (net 10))
 (segment (start 46.096 42.54) (end 50.29 42.54) (width 0.2) (layer "B.Cu") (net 10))
 (segment (start 45.974 42.418) (end 46.096 42.54) (width 0.2) (layer "B.Cu") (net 10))
 (segment (start 60.13 57) (end 60.13 62.14) (width 0.2) (layer "F.Cu") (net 1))
 (segment (start 60.13 62.14) (end 59.88 62.39) (width 0.2) (layer "F.Cu") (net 1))
 (segment (start 56.905 71.055) (end 59.76 68.2) (width 0.2) (layer "B.Cu") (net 1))
 (segment (start 56.905 80.55) (end 56.905 71.055) (width 0.2) (layer "B.Cu") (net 1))
 (segment (start 59.88 62.39) (end 59.88 68.08) (width 0.2) (layer "B.Cu") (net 1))
 (segment (start 59.88 68.08) (end 59.76 68.2) (width 0.2) (layer "B.Cu") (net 1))
 (segment (start 61.13 57) (end 61.13 61.1) (width 0.2) (layer "F.Cu") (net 2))
 (segment (start 61.13 61.1) (end 62.42 62.39) (width 0.2) (layer "F.Cu") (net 2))
 (segment (start 59.445 80.55) (end 59.445 71.055) (width 0.2) (layer "B.Cu") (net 2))
 (segment (start 62.3 68.2) (end 62.3 62.51) (width 0.2) (layer "B.Cu") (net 2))
 (segment (start 62.3 62.51) (end 62.42 62.39) (width 0.2) (layer "B.Cu") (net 2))
 (segment (start 59.445 71.055) (end 62.3 68.2) (width 0.2) (layer "B.Cu") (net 2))
 (segment (start 62.13 57) (end 62.13 59.56) (width 0.2) (layer "F.Cu") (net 3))
 (segment (start 62.13 59.56) (end 64.96 62.39) (width 0.2) (layer "F.Cu") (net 3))
 (segment (start 61.985 80.55) (end 61.985 71.055) (width 0.2) (layer "B.Cu") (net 3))
 (segment (start 61.985 71.055) (end 64.84 68.2) (width 0.2) (layer "B.Cu") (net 3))
 (segment (start 64.96 68.08) (end 64.84 68.2) (width 0.2) (layer "B.Cu") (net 3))
 (segment (start 64.96 62.39) (end 64.96 68.08) (width 0.2) (layer "B.Cu") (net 3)))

